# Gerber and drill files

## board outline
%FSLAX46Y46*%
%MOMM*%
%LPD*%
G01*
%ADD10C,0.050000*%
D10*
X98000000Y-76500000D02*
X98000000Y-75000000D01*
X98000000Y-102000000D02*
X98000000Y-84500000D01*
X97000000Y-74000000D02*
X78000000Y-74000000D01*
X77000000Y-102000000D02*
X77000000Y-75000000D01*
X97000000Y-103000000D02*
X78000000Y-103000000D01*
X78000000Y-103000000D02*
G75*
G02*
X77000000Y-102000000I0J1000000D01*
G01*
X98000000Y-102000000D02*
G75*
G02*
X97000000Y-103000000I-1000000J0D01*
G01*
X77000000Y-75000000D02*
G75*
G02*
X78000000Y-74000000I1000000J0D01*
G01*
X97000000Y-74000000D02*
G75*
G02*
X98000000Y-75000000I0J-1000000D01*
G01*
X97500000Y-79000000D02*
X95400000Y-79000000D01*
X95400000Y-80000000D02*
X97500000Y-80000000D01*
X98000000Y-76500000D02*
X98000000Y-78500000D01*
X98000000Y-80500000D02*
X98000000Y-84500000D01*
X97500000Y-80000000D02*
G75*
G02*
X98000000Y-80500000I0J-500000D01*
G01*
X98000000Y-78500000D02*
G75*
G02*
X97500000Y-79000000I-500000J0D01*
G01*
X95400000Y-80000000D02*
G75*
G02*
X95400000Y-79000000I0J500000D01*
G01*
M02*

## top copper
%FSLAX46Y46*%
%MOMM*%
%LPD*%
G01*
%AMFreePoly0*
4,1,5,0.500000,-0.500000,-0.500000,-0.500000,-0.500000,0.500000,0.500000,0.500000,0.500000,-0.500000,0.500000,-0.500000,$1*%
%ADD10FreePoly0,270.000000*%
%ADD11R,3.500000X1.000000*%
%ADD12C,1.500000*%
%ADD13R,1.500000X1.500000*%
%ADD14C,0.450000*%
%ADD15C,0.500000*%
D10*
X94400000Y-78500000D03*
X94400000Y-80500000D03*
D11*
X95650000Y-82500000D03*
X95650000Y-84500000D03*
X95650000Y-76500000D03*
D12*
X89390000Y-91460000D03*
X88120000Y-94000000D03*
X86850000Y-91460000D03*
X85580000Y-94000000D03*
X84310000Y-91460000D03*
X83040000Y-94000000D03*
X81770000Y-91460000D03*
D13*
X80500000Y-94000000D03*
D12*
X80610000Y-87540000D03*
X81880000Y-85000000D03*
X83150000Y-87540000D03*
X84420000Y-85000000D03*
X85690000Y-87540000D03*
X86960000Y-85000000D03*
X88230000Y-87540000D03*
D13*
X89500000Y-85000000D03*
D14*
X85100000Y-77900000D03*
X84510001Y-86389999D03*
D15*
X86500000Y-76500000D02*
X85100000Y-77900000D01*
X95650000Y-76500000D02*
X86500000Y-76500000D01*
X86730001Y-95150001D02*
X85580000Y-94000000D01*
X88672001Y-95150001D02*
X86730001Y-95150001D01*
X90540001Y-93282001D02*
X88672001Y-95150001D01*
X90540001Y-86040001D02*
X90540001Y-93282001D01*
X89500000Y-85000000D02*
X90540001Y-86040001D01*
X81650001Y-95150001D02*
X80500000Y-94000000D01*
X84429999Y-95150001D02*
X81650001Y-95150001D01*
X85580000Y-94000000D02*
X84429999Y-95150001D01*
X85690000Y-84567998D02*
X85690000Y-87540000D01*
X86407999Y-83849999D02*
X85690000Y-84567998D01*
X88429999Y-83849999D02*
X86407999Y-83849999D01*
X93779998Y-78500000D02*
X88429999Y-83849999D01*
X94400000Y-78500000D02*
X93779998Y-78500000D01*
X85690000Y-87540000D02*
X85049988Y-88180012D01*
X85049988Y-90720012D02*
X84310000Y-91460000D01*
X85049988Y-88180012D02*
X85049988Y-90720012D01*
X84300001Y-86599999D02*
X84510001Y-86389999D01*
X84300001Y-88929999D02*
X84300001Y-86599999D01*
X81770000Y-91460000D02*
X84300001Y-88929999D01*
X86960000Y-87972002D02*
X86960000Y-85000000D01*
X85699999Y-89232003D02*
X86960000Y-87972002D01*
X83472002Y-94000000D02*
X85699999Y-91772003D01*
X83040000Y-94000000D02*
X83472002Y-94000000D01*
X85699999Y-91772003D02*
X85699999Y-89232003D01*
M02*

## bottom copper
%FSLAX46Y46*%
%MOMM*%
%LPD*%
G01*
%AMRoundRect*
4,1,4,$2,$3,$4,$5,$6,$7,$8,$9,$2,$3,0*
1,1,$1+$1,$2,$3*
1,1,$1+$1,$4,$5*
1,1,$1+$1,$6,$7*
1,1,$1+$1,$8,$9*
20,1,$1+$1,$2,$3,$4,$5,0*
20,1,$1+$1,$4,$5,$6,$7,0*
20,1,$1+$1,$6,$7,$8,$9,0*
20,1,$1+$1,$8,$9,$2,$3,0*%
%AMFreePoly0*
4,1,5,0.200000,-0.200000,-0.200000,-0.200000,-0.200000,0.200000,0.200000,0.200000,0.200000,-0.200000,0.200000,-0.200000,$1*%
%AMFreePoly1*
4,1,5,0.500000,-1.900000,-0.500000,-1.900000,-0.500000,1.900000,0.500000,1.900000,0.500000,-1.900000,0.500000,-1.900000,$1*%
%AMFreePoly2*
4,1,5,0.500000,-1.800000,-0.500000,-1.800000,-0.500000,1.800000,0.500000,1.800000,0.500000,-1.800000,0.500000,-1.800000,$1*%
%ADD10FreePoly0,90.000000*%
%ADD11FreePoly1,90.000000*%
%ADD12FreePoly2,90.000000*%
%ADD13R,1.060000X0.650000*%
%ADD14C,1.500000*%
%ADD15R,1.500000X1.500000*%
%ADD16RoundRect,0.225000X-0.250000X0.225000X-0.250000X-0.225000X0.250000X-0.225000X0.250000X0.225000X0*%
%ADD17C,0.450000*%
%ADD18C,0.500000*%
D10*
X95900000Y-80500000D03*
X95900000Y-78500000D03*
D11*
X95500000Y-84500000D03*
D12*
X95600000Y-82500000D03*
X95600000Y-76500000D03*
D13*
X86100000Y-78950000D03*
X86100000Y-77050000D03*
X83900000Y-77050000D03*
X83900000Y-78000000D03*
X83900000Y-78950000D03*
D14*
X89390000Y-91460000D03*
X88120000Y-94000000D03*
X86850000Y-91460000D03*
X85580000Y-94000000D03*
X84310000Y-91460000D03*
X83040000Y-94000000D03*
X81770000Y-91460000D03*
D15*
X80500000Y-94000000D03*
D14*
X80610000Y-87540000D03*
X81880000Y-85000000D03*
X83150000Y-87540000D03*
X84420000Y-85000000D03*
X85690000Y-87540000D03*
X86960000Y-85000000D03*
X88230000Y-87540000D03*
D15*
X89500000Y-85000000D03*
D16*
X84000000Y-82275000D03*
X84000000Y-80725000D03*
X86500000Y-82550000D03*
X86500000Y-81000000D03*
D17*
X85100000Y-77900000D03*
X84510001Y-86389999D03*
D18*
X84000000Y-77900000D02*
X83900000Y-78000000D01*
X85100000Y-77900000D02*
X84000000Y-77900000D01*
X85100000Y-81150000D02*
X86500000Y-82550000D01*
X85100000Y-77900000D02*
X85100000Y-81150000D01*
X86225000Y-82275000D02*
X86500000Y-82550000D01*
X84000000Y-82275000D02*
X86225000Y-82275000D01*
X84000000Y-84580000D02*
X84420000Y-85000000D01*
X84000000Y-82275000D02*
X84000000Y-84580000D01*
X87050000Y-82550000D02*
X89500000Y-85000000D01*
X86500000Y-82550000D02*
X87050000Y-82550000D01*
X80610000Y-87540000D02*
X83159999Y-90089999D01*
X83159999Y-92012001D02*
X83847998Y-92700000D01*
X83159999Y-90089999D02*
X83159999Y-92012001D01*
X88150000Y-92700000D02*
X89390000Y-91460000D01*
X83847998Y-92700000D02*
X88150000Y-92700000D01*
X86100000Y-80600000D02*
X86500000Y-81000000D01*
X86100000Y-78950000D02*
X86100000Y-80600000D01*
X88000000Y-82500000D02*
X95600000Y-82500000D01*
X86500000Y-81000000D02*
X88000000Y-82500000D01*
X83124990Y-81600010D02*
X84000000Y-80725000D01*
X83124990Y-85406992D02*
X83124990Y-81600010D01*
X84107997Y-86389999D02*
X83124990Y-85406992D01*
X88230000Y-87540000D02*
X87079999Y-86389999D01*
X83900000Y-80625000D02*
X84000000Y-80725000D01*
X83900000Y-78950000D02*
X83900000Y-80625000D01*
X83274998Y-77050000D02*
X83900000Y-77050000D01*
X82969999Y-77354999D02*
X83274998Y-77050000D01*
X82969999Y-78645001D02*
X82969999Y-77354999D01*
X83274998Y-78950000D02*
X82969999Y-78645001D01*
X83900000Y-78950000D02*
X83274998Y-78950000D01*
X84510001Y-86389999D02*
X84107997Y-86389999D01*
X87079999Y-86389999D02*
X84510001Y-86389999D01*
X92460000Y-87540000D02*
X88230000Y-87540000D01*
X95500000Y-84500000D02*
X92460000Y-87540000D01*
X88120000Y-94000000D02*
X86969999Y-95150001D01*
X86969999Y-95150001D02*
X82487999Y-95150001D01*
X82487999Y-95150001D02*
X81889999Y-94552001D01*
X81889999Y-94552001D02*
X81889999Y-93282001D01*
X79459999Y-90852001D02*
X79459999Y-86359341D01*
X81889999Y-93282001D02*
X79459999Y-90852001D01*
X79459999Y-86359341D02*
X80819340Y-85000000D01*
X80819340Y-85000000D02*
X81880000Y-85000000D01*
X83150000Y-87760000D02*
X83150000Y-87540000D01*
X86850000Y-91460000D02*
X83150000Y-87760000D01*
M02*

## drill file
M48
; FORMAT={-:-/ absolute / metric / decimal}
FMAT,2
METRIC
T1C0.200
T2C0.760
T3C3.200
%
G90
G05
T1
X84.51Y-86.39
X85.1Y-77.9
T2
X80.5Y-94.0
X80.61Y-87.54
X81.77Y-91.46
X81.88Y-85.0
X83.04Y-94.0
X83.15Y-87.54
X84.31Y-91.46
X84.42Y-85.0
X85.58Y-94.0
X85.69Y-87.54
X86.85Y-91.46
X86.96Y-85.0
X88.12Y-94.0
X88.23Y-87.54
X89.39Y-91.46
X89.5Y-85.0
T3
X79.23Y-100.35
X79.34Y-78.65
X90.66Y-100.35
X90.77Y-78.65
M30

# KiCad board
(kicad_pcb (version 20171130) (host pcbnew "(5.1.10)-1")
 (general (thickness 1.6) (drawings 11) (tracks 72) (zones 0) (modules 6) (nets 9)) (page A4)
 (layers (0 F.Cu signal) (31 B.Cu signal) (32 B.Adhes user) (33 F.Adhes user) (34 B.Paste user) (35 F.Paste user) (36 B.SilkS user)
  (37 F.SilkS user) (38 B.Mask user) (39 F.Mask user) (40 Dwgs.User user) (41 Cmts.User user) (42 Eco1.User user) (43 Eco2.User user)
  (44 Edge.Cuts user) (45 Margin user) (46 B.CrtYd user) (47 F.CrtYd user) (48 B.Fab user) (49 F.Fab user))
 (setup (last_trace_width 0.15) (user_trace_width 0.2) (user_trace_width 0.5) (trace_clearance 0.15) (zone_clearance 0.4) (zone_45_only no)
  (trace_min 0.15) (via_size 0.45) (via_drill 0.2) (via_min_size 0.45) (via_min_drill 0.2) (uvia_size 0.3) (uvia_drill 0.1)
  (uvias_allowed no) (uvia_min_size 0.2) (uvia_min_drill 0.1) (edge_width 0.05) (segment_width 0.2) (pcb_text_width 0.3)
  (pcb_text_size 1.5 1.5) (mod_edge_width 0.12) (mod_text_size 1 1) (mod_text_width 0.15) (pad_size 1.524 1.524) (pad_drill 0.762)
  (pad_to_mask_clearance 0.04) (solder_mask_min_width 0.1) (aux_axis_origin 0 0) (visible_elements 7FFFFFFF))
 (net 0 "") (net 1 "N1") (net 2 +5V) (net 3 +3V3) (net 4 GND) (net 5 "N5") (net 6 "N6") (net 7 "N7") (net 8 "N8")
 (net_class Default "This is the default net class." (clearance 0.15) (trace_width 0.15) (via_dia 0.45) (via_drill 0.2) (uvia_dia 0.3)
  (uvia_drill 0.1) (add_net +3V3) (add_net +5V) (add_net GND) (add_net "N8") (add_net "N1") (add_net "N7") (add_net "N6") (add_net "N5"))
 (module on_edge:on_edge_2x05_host (layer F.Cu) (at 98 80.5 270)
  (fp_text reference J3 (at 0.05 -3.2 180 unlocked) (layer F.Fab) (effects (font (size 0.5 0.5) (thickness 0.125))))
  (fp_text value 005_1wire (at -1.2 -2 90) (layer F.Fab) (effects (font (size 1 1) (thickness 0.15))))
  (fp_line (start -1.5 0.5) (end -1.5 2.6) (layer Edge.Cuts) (width 0.05))
  (fp_line (start -0.5 2.6) (end -0.5 0.5) (layer Edge.Cuts) (width 0.05))
  (fp_line (start -4 0) (end -2 0) (layer Edge.Cuts) (width 0.05))
  (fp_line (start 0 0) (end 4 0) (layer Edge.Cuts) (width 0.05))
  (fp_arc (start 0 0.5) (end 0 0) (angle -90) (layer Edge.Cuts) (width 0.05))
  (fp_arc (start -2 0.5) (end -1.5 0.5) (angle -90) (layer Edge.Cuts) (width 0.05))
  (fp_arc (start -1 2.6) (end -1.5 2.6) (angle -180) (layer Edge.Cuts) (width 0.05))
  (pad 2 smd custom (at -2 3.6 270) (size 1 1) (layers F.Cu F.Mask) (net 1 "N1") (zone_connect 0)
   (options (clearance outline) (anchor rect)) (primitives))
  (pad 3 smd custom (at 0 3.6 270) (size 1 1) (layers F.Cu F.Mask) (zone_connect 0) (options (clearance outline) (anchor rect)) (primitives))
  (pad 8 smd custom (at 0 2.1 90) (size 0.4 0.4) (layers B.Cu B.Mask) (zone_connect 0) (options (clearance outline) (anchor rect))
   (primitives))
  (pad 7 smd custom (at -2 2.1 90) (size 0.4 0.4) (layers B.Cu B.Mask) (zone_connect 0) (options (clearance outline) (anchor rect))
   (primitives))
  (pad 4 smd rect (at 2 2.35 270) (size 1 3.5) (layers F.Cu F.Mask) (zone_connect 0))
  (pad 10 smd custom (at 4 2.5 90) (size 1 3.8) (layers B.Cu B.Mask) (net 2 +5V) (zone_connect 0)
   (options (clearance outline) (anchor rect)) (primitives))
  (pad 9 smd custom (at 2 2.4 90) (size 1 3.6) (layers B.Cu B.Mask) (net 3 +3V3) (zone_connect 0)
   (options (clearance outline) (anchor rect)) (primitives))
  (pad 6 smd custom (at -4 2.4 90) (size 1 3.6) (layers B.Cu B.Mask) (zone_connect 0) (options (clearance outline) (anchor rect))
   (primitives))
  (pad 5 smd rect (at 4 2.35 270) (size 1 3.5) (layers F.Cu F.Mask) (zone_connect 0))
  (pad 1 smd rect (at -4 2.35 270) (size 1 3.5) (layers F.Cu F.Mask) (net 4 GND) (zone_connect 0)))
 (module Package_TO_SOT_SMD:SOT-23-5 (layer B.Cu) (at 85 78)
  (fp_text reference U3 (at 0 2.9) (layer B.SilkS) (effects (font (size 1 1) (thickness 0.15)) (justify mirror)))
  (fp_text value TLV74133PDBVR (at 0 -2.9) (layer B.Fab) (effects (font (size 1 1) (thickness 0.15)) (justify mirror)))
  (pad 5 smd rect (at 1.1 0.95) (size 1.06 0.65) (layers B.Cu B.Paste B.Mask) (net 3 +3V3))
  (pad 4 smd rect (at 1.1 -0.95) (size 1.06 0.65) (layers B.Cu B.Paste B.Mask))
  (pad 3 smd rect (at -1.1 -0.95) (size 1.06 0.65) (layers B.Cu B.Paste B.Mask) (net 2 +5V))
  (pad 2 smd rect (at -1.1 0) (size 1.06 0.65) (layers B.Cu B.Paste B.Mask) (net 4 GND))
  (pad 1 smd rect (at -1.1 0.95) (size 1.06 0.65) (layers B.Cu B.Paste B.Mask) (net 2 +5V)))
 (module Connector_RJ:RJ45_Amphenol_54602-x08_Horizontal (layer F.Cu) (at 80.5 94)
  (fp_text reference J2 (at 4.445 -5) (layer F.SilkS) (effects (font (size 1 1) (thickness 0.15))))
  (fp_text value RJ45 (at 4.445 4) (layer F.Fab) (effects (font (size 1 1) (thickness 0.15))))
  (pad 8 thru_hole circle (at 8.89 -2.54) (size 1.5 1.5) (drill 0.76) (layers *.Cu *.Mask) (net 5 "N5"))
  (pad 7 thru_hole circle (at 7.62 0) (size 1.5 1.5) (drill 0.76) (layers *.Cu *.Mask) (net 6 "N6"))
  (pad 6 thru_hole circle (at 6.35 -2.54) (size 1.5 1.5) (drill 0.76) (layers *.Cu *.Mask) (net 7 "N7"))
  (pad 5 thru_hole circle (at 5.08 0) (size 1.5 1.5) (drill 0.76) (layers *.Cu *.Mask) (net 4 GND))
  (pad 4 thru_hole circle (at 3.81 -2.54) (size 1.5 1.5) (drill 0.76) (layers *.Cu *.Mask) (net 1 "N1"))
  (pad 3 thru_hole circle (at 2.54 0) (size 1.5 1.5) (drill 0.76) (layers *.Cu *.Mask) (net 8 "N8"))
  (pad 2 thru_hole circle (at 1.27 -2.54) (size 1.5 1.5) (drill 0.76) (layers *.Cu *.Mask) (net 2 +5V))
  (pad 1 thru_hole rect (at 0 0) (size 1.5 1.5) (drill 0.76) (layers *.Cu *.Mask) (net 4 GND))
  (pad "" np_thru_hole circle (at -1.27 6.35) (size 3.2 3.2) (drill 3.2) (layers *.Cu *.Mask))
  (pad "" np_thru_hole circle (at 10.16 6.35) (size 3.2 3.2) (drill 3.2) (layers *.Cu *.Mask)))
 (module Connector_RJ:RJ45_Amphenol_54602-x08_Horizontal (layer F.Cu) (at 89.5 85 180)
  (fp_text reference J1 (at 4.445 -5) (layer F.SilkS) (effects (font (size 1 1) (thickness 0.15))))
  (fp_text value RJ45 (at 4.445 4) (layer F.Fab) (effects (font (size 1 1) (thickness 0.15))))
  (pad 8 thru_hole circle (at 8.89 -2.54 180) (size 1.5 1.5) (drill 0.76) (layers *.Cu *.Mask) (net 5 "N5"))
  (pad 7 thru_hole circle (at 7.62 0 180) (size 1.5 1.5) (drill 0.76) (layers *.Cu *.Mask) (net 6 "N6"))
  (pad 6 thru_hole circle (at 6.35 -2.54 180) (size 1.5 1.5) (drill 0.76) (layers *.Cu *.Mask) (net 7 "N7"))
  (pad 5 thru_hole circle (at 5.08 0 180) (size 1.5 1.5) (drill 0.76) (layers *.Cu *.Mask) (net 4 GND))
  (pad 4 thru_hole circle (at 3.81 -2.54 180) (size 1.5 1.5) (drill 0.76) (layers *.Cu *.Mask) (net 1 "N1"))
  (pad 3 thru_hole circle (at 2.54 0 180) (size 1.5 1.5) (drill 0.76) (layers *.Cu *.Mask) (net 8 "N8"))
  (pad 2 thru_hole circle (at 1.27 -2.54 180) (size 1.5 1.5) (drill 0.76) (layers *.Cu *.Mask) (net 2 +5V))
  (pad 1 thru_hole rect (at 0 0 180) (size 1.5 1.5) (drill 0.76) (layers *.Cu *.Mask) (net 4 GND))
  (pad "" np_thru_hole circle (at -1.27 6.35 180) (size 3.2 3.2) (drill 3.2) (layers *.Cu *.Mask))
  (pad "" np_thru_hole circle (at 10.16 6.35 180) (size 3.2 3.2) (drill 3.2) (layers *.Cu *.Mask)))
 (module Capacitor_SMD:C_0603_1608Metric (layer B.Cu) (at 84 81.5 270)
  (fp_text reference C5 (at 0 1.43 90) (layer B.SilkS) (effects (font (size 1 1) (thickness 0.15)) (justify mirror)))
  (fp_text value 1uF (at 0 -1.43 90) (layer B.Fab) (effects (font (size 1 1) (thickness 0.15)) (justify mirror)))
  (pad 2 smd roundrect (at 0.775 0 270) (size 0.9 0.95) (layers B.Cu B.Paste B.Mask) (roundrect_rratio 0.25) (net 4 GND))
  (pad 1 smd roundrect (at -0.775 0 270) (size 0.9 0.95) (layers B.Cu B.Paste B.Mask) (roundrect_rratio 0.25) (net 2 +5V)))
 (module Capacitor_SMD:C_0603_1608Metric (layer B.Cu) (at 86.5 81.775 270)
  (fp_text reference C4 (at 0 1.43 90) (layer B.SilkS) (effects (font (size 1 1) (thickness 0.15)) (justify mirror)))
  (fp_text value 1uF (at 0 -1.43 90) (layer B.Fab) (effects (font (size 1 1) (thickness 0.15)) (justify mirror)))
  (pad 2 smd roundrect (at 0.775 0 270) (size 0.9 0.95) (layers B.Cu B.Paste B.Mask) (roundrect_rratio 0.25) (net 4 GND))
  (pad 1 smd roundrect (at -0.775 0 270) (size 0.9 0.95) (layers B.Cu B.Paste B.Mask) (roundrect_rratio 0.25) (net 3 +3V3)))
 (gr_line (start 98 76.5) (end 98 75) (layer Edge.Cuts) (width 0.05))
 (gr_line (start 98 102) (end 98 84.5) (layer Edge.Cuts) (width 0.05))
 (gr_line (start 97 74) (end 78 74) (layer Edge.Cuts) (width 0.05))
 (gr_line (start 77 102) (end 77 75) (layer Edge.Cuts) (width 0.05))
 (gr_line (start 97 103) (end 78 103) (layer Edge.Cuts) (width 0.05))
 (gr_arc (start 78 102) (end 77 102) (angle -90) (layer Edge.Cuts) (width 0.05))
 (gr_arc (start 97 102) (end 97 103) (angle -90) (layer Edge.Cuts) (width 0.05))
 (gr_arc (start 78 75) (end 78 74) (angle -90) (layer Edge.Cuts) (width 0.05))
 (gr_arc (start 97 75) (end 98 75) (angle -90) (layer Edge.Cuts) (width 0.05))
 (via (at 85.1 77.9) (size 0.45) (drill 0.2) (layers F.Cu B.Cu) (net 4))
 (segment (start 86.5 76.5) (end 85.1 77.9) (width 0.5) (layer F.Cu) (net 4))
 (segment (start 95.65 76.5) (end 86.5 76.5) (width 0.5) (layer F.Cu) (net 4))
 (segment (start 84 77.9) (end 83.9 78) (width 0.5) (layer B.Cu) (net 4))
 (segment (start 85.1 77.9) (end 84 77.9) (width 0.5) (layer B.Cu) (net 4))
 (segment (start 85.1 81.15) (end 86.5 82.55) (width 0.5) (layer B.Cu) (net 4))
 (segment (start 85.1 77.9) (end 85.1 81.15) (width 0.5) (layer B.Cu) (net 4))
 (segment (start 86.225 82.275) (end 86.5 82.55) (width 0.5) (layer B.Cu) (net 4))
 (segment (start 84 82.275) (end 86.225 82.275) (width 0.5) (layer B.Cu) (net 4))
 (segment (start 84 84.58) (end 84.42 85) (width 0.5) (layer B.Cu) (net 4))
 (segment (start 84 82.275) (end 84 84.58) (width 0.5) (layer B.Cu) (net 4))
 (segment (start 87.05 82.55) (end 89.5 85) (width 0.5) (layer B.Cu) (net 4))
 (segment (start 86.5 82.55) (end 87.05 82.55) (width 0.5) (layer B.Cu) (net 4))
 (segment (start 86.730001 95.150001) (end 85.58 94) (width 0.5) (layer F.Cu) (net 4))
 (segment (start 88.672001 95.150001) (end 86.730001 95.150001) (width 0.5) (layer F.Cu) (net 4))
 (segment (start 90.540001 93.282001) (end 88.672001 95.150001) (width 0.5) (layer F.Cu) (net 4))
 (segment (start 90.540001 86.040001) (end 90.540001 93.282001) (width 0.5) (layer F.Cu) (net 4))
 (segment (start 89.5 85) (end 90.540001 86.040001) (width 0.5) (layer F.Cu) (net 4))
 (segment (start 81.650001 95.150001) (end 80.5 94) (width 0.5) (layer F.Cu) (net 4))
 (segment (start 84.429999 95.150001) (end 81.650001 95.150001) (width 0.5) (layer F.Cu) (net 4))
 (segment (start 85.58 94) (end 84.429999 95.150001) (width 0.5) (layer F.Cu) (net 4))
 (segment (start 80.61 87.54) (end 83.159999 90.089999) (width 0.5) (layer B.Cu) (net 5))
 (segment (start 83.159999 92.012001) (end 83.847998 92.7) (width 0.5) (layer B.Cu) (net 5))
 (segment (start 83.159999 90.089999) (end 83.159999 92.012001) (width 0.5) (layer B.Cu) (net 5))
 (segment (start 88.15 92.7) (end 89.39 91.46) (width 0.5) (layer B.Cu) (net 5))
 (segment (start 83.847998 92.7) (end 88.15 92.7) (width 0.5) (layer B.Cu) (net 5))
 (segment (start 85.69 84.567998) (end 85.69 87.54) (width 0.5) (layer F.Cu) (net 1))
 (segment (start 86.407999 83.849999) (end 85.69 84.567998) (width 0.5) (layer F.Cu) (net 1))
 (segment (start 88.429999 83.849999) (end 86.407999 83.849999) (width 0.5) (layer F.Cu) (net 1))
 (segment (start 93.779998 78.5) (end 88.429999 83.849999) (width 0.5) (layer F.Cu) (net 1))
 (segment (start 94.4 78.5) (end 93.779998 78.5) (width 0.5) (layer F.Cu) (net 1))
 (segment (start 85.69 87.54) (end 85.049988 88.180012) (width 0.5) (layer F.Cu) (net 1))
 (segment (start 85.049988 90.720012) (end 84.31 91.46) (width 0.5) (layer F.Cu) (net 1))
 (segment (start 85.049988 88.180012) (end 85.049988 90.720012) (width 0.5) (layer F.Cu) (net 1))
 (segment (start 86.1 80.6) (end 86.5 81) (width 0.5) (layer B.Cu) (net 3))
 (segment (start 86.1 78.95) (end 86.1 80.6) (width 0.5) (layer B.Cu) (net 3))
 (segment (start 88 82.5) (end 95.6 82.5) (width 0.5) (layer B.Cu) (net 3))
 (segment (start 86.5 81) (end 88 82.5) (width 0.5) (layer B.Cu) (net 3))
 (segment (start 83.12499 81.60001) (end 84 80.725) (width 0.5) (layer B.Cu) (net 2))
 (segment (start 83.12499 85.406992) (end 83.12499 81.60001) (width 0.5) (layer B.Cu) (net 2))
 (segment (start 84.107997 86.389999) (end 83.12499 85.406992) (width 0.5) (layer B.Cu) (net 2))
 (segment (start 88.23 87.54) (end 87.079999 86.389999) (width 0.5) (layer B.Cu) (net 2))
 (segment (start 83.9 80.625) (end 84 80.725) (width 0.5) (layer B.Cu) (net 2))
 (segment (start 83.9 78.95) (end 83.9 80.625) (width 0.5) (layer B.Cu) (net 2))
 (segment (start 83.274998 77.05) (end 83.9 77.05) (width 0.5) (layer B.Cu) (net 2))
 (segment (start 82.969999 77.354999) (end 83.274998 77.05) (width 0.5) (layer B.Cu) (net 2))
 (segment (start 82.969999 78.645001) (end 82.969999 77.354999) (width 0.5) (layer B.Cu) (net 2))
 (segment (start 83.274998 78.95) (end 82.969999 78.645001) (width 0.5) (layer B.Cu) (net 2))
 (segment (start 83.9 78.95) (end 83.274998 78.95) (width 0.5) (layer B.Cu) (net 2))
 (segment (start 84.300001 86.599999) (end 84.510001 86.389999) (width 0.5) (layer F.Cu) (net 2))
 (via (at 84.510001 86.389999) (size 0.45) (drill 0.2) (layers F.Cu B.Cu) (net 2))
 (segment (start 84.300001 88.929999) (end 84.300001 86.599999) (width 0.5) (layer F.Cu) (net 2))
 (segment (start 81.77 91.46) (end 84.300001 88.929999) (width 0.5) (layer F.Cu) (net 2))
 (segment (start 84.510001 86.389999) (end 84.107997 86.389999) (width 0.5) (layer B.Cu) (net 2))
 (segment (start 87.079999 86.389999) (end 84.510001 86.389999) (width 0.5) (layer B.Cu) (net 2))
 (segment (start 92.46 87.54) (end 88.23 87.54) (width 0.5) (layer B.Cu) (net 2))
 (segment (start 95.5 84.5) (end 92.46 87.54) (width 0.5) (layer B.Cu) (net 2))
 (segment (start 88.12 94) (end 86.969999 95.150001) (width 0.5) (layer B.Cu) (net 6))
 (segment (start 86.969999 95.150001) (end 82.487999 95.150001) (width 0.5) (layer B.Cu) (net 6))
 (segment (start 82.487999 95.150001) (end 81.889999 94.552001) (width 0.5) (layer B.Cu) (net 6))
 (segment (start 81.889999 94.552001) (end 81.889999 93.282001) (width 0.5) (layer B.Cu) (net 6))
 (segment (start 79.459999 90.852001) (end 79.459999 86.359341) (width 0.5) (layer B.Cu) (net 6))
 (segment (start 81.889999 93.282001) (end 79.459999 90.852001) (width 0.5) (layer B.Cu) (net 6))
 (segment (start 79.459999 86.359341) (end 80.81934 85) (width 0.5) (layer B.Cu) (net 6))
 (segment (start 80.81934 85) (end 81.88 85) (width 0.5) (layer B.Cu) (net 6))
 (segment (start 83.15 87.76) (end 83.15 87.54) (width 0.5) (layer B.Cu) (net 7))
 (segment (start 86.85 91.46) (end 83.15 87.76) (width 0.5) (layer B.Cu) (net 7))
 (segment (start 86.96 87.972002) (end 86.96 85) (width 0.5) (layer F.Cu) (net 8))
 (segment (start 85.699999 89.232003) (end 86.96 87.972002) (width 0.5) (layer F.Cu) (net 8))
 (segment (start 83.472002 94) (end 85.699999 91.772003) (width 0.5) (layer F.Cu) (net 8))
 (segment (start 83.04 94) (end 83.472002 94) (width 0.5) (layer F.Cu) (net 8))
 (segment (start 85.699999 91.772003) (end 85.699999 89.232003) (width 0.5) (layer F.Cu) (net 8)))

